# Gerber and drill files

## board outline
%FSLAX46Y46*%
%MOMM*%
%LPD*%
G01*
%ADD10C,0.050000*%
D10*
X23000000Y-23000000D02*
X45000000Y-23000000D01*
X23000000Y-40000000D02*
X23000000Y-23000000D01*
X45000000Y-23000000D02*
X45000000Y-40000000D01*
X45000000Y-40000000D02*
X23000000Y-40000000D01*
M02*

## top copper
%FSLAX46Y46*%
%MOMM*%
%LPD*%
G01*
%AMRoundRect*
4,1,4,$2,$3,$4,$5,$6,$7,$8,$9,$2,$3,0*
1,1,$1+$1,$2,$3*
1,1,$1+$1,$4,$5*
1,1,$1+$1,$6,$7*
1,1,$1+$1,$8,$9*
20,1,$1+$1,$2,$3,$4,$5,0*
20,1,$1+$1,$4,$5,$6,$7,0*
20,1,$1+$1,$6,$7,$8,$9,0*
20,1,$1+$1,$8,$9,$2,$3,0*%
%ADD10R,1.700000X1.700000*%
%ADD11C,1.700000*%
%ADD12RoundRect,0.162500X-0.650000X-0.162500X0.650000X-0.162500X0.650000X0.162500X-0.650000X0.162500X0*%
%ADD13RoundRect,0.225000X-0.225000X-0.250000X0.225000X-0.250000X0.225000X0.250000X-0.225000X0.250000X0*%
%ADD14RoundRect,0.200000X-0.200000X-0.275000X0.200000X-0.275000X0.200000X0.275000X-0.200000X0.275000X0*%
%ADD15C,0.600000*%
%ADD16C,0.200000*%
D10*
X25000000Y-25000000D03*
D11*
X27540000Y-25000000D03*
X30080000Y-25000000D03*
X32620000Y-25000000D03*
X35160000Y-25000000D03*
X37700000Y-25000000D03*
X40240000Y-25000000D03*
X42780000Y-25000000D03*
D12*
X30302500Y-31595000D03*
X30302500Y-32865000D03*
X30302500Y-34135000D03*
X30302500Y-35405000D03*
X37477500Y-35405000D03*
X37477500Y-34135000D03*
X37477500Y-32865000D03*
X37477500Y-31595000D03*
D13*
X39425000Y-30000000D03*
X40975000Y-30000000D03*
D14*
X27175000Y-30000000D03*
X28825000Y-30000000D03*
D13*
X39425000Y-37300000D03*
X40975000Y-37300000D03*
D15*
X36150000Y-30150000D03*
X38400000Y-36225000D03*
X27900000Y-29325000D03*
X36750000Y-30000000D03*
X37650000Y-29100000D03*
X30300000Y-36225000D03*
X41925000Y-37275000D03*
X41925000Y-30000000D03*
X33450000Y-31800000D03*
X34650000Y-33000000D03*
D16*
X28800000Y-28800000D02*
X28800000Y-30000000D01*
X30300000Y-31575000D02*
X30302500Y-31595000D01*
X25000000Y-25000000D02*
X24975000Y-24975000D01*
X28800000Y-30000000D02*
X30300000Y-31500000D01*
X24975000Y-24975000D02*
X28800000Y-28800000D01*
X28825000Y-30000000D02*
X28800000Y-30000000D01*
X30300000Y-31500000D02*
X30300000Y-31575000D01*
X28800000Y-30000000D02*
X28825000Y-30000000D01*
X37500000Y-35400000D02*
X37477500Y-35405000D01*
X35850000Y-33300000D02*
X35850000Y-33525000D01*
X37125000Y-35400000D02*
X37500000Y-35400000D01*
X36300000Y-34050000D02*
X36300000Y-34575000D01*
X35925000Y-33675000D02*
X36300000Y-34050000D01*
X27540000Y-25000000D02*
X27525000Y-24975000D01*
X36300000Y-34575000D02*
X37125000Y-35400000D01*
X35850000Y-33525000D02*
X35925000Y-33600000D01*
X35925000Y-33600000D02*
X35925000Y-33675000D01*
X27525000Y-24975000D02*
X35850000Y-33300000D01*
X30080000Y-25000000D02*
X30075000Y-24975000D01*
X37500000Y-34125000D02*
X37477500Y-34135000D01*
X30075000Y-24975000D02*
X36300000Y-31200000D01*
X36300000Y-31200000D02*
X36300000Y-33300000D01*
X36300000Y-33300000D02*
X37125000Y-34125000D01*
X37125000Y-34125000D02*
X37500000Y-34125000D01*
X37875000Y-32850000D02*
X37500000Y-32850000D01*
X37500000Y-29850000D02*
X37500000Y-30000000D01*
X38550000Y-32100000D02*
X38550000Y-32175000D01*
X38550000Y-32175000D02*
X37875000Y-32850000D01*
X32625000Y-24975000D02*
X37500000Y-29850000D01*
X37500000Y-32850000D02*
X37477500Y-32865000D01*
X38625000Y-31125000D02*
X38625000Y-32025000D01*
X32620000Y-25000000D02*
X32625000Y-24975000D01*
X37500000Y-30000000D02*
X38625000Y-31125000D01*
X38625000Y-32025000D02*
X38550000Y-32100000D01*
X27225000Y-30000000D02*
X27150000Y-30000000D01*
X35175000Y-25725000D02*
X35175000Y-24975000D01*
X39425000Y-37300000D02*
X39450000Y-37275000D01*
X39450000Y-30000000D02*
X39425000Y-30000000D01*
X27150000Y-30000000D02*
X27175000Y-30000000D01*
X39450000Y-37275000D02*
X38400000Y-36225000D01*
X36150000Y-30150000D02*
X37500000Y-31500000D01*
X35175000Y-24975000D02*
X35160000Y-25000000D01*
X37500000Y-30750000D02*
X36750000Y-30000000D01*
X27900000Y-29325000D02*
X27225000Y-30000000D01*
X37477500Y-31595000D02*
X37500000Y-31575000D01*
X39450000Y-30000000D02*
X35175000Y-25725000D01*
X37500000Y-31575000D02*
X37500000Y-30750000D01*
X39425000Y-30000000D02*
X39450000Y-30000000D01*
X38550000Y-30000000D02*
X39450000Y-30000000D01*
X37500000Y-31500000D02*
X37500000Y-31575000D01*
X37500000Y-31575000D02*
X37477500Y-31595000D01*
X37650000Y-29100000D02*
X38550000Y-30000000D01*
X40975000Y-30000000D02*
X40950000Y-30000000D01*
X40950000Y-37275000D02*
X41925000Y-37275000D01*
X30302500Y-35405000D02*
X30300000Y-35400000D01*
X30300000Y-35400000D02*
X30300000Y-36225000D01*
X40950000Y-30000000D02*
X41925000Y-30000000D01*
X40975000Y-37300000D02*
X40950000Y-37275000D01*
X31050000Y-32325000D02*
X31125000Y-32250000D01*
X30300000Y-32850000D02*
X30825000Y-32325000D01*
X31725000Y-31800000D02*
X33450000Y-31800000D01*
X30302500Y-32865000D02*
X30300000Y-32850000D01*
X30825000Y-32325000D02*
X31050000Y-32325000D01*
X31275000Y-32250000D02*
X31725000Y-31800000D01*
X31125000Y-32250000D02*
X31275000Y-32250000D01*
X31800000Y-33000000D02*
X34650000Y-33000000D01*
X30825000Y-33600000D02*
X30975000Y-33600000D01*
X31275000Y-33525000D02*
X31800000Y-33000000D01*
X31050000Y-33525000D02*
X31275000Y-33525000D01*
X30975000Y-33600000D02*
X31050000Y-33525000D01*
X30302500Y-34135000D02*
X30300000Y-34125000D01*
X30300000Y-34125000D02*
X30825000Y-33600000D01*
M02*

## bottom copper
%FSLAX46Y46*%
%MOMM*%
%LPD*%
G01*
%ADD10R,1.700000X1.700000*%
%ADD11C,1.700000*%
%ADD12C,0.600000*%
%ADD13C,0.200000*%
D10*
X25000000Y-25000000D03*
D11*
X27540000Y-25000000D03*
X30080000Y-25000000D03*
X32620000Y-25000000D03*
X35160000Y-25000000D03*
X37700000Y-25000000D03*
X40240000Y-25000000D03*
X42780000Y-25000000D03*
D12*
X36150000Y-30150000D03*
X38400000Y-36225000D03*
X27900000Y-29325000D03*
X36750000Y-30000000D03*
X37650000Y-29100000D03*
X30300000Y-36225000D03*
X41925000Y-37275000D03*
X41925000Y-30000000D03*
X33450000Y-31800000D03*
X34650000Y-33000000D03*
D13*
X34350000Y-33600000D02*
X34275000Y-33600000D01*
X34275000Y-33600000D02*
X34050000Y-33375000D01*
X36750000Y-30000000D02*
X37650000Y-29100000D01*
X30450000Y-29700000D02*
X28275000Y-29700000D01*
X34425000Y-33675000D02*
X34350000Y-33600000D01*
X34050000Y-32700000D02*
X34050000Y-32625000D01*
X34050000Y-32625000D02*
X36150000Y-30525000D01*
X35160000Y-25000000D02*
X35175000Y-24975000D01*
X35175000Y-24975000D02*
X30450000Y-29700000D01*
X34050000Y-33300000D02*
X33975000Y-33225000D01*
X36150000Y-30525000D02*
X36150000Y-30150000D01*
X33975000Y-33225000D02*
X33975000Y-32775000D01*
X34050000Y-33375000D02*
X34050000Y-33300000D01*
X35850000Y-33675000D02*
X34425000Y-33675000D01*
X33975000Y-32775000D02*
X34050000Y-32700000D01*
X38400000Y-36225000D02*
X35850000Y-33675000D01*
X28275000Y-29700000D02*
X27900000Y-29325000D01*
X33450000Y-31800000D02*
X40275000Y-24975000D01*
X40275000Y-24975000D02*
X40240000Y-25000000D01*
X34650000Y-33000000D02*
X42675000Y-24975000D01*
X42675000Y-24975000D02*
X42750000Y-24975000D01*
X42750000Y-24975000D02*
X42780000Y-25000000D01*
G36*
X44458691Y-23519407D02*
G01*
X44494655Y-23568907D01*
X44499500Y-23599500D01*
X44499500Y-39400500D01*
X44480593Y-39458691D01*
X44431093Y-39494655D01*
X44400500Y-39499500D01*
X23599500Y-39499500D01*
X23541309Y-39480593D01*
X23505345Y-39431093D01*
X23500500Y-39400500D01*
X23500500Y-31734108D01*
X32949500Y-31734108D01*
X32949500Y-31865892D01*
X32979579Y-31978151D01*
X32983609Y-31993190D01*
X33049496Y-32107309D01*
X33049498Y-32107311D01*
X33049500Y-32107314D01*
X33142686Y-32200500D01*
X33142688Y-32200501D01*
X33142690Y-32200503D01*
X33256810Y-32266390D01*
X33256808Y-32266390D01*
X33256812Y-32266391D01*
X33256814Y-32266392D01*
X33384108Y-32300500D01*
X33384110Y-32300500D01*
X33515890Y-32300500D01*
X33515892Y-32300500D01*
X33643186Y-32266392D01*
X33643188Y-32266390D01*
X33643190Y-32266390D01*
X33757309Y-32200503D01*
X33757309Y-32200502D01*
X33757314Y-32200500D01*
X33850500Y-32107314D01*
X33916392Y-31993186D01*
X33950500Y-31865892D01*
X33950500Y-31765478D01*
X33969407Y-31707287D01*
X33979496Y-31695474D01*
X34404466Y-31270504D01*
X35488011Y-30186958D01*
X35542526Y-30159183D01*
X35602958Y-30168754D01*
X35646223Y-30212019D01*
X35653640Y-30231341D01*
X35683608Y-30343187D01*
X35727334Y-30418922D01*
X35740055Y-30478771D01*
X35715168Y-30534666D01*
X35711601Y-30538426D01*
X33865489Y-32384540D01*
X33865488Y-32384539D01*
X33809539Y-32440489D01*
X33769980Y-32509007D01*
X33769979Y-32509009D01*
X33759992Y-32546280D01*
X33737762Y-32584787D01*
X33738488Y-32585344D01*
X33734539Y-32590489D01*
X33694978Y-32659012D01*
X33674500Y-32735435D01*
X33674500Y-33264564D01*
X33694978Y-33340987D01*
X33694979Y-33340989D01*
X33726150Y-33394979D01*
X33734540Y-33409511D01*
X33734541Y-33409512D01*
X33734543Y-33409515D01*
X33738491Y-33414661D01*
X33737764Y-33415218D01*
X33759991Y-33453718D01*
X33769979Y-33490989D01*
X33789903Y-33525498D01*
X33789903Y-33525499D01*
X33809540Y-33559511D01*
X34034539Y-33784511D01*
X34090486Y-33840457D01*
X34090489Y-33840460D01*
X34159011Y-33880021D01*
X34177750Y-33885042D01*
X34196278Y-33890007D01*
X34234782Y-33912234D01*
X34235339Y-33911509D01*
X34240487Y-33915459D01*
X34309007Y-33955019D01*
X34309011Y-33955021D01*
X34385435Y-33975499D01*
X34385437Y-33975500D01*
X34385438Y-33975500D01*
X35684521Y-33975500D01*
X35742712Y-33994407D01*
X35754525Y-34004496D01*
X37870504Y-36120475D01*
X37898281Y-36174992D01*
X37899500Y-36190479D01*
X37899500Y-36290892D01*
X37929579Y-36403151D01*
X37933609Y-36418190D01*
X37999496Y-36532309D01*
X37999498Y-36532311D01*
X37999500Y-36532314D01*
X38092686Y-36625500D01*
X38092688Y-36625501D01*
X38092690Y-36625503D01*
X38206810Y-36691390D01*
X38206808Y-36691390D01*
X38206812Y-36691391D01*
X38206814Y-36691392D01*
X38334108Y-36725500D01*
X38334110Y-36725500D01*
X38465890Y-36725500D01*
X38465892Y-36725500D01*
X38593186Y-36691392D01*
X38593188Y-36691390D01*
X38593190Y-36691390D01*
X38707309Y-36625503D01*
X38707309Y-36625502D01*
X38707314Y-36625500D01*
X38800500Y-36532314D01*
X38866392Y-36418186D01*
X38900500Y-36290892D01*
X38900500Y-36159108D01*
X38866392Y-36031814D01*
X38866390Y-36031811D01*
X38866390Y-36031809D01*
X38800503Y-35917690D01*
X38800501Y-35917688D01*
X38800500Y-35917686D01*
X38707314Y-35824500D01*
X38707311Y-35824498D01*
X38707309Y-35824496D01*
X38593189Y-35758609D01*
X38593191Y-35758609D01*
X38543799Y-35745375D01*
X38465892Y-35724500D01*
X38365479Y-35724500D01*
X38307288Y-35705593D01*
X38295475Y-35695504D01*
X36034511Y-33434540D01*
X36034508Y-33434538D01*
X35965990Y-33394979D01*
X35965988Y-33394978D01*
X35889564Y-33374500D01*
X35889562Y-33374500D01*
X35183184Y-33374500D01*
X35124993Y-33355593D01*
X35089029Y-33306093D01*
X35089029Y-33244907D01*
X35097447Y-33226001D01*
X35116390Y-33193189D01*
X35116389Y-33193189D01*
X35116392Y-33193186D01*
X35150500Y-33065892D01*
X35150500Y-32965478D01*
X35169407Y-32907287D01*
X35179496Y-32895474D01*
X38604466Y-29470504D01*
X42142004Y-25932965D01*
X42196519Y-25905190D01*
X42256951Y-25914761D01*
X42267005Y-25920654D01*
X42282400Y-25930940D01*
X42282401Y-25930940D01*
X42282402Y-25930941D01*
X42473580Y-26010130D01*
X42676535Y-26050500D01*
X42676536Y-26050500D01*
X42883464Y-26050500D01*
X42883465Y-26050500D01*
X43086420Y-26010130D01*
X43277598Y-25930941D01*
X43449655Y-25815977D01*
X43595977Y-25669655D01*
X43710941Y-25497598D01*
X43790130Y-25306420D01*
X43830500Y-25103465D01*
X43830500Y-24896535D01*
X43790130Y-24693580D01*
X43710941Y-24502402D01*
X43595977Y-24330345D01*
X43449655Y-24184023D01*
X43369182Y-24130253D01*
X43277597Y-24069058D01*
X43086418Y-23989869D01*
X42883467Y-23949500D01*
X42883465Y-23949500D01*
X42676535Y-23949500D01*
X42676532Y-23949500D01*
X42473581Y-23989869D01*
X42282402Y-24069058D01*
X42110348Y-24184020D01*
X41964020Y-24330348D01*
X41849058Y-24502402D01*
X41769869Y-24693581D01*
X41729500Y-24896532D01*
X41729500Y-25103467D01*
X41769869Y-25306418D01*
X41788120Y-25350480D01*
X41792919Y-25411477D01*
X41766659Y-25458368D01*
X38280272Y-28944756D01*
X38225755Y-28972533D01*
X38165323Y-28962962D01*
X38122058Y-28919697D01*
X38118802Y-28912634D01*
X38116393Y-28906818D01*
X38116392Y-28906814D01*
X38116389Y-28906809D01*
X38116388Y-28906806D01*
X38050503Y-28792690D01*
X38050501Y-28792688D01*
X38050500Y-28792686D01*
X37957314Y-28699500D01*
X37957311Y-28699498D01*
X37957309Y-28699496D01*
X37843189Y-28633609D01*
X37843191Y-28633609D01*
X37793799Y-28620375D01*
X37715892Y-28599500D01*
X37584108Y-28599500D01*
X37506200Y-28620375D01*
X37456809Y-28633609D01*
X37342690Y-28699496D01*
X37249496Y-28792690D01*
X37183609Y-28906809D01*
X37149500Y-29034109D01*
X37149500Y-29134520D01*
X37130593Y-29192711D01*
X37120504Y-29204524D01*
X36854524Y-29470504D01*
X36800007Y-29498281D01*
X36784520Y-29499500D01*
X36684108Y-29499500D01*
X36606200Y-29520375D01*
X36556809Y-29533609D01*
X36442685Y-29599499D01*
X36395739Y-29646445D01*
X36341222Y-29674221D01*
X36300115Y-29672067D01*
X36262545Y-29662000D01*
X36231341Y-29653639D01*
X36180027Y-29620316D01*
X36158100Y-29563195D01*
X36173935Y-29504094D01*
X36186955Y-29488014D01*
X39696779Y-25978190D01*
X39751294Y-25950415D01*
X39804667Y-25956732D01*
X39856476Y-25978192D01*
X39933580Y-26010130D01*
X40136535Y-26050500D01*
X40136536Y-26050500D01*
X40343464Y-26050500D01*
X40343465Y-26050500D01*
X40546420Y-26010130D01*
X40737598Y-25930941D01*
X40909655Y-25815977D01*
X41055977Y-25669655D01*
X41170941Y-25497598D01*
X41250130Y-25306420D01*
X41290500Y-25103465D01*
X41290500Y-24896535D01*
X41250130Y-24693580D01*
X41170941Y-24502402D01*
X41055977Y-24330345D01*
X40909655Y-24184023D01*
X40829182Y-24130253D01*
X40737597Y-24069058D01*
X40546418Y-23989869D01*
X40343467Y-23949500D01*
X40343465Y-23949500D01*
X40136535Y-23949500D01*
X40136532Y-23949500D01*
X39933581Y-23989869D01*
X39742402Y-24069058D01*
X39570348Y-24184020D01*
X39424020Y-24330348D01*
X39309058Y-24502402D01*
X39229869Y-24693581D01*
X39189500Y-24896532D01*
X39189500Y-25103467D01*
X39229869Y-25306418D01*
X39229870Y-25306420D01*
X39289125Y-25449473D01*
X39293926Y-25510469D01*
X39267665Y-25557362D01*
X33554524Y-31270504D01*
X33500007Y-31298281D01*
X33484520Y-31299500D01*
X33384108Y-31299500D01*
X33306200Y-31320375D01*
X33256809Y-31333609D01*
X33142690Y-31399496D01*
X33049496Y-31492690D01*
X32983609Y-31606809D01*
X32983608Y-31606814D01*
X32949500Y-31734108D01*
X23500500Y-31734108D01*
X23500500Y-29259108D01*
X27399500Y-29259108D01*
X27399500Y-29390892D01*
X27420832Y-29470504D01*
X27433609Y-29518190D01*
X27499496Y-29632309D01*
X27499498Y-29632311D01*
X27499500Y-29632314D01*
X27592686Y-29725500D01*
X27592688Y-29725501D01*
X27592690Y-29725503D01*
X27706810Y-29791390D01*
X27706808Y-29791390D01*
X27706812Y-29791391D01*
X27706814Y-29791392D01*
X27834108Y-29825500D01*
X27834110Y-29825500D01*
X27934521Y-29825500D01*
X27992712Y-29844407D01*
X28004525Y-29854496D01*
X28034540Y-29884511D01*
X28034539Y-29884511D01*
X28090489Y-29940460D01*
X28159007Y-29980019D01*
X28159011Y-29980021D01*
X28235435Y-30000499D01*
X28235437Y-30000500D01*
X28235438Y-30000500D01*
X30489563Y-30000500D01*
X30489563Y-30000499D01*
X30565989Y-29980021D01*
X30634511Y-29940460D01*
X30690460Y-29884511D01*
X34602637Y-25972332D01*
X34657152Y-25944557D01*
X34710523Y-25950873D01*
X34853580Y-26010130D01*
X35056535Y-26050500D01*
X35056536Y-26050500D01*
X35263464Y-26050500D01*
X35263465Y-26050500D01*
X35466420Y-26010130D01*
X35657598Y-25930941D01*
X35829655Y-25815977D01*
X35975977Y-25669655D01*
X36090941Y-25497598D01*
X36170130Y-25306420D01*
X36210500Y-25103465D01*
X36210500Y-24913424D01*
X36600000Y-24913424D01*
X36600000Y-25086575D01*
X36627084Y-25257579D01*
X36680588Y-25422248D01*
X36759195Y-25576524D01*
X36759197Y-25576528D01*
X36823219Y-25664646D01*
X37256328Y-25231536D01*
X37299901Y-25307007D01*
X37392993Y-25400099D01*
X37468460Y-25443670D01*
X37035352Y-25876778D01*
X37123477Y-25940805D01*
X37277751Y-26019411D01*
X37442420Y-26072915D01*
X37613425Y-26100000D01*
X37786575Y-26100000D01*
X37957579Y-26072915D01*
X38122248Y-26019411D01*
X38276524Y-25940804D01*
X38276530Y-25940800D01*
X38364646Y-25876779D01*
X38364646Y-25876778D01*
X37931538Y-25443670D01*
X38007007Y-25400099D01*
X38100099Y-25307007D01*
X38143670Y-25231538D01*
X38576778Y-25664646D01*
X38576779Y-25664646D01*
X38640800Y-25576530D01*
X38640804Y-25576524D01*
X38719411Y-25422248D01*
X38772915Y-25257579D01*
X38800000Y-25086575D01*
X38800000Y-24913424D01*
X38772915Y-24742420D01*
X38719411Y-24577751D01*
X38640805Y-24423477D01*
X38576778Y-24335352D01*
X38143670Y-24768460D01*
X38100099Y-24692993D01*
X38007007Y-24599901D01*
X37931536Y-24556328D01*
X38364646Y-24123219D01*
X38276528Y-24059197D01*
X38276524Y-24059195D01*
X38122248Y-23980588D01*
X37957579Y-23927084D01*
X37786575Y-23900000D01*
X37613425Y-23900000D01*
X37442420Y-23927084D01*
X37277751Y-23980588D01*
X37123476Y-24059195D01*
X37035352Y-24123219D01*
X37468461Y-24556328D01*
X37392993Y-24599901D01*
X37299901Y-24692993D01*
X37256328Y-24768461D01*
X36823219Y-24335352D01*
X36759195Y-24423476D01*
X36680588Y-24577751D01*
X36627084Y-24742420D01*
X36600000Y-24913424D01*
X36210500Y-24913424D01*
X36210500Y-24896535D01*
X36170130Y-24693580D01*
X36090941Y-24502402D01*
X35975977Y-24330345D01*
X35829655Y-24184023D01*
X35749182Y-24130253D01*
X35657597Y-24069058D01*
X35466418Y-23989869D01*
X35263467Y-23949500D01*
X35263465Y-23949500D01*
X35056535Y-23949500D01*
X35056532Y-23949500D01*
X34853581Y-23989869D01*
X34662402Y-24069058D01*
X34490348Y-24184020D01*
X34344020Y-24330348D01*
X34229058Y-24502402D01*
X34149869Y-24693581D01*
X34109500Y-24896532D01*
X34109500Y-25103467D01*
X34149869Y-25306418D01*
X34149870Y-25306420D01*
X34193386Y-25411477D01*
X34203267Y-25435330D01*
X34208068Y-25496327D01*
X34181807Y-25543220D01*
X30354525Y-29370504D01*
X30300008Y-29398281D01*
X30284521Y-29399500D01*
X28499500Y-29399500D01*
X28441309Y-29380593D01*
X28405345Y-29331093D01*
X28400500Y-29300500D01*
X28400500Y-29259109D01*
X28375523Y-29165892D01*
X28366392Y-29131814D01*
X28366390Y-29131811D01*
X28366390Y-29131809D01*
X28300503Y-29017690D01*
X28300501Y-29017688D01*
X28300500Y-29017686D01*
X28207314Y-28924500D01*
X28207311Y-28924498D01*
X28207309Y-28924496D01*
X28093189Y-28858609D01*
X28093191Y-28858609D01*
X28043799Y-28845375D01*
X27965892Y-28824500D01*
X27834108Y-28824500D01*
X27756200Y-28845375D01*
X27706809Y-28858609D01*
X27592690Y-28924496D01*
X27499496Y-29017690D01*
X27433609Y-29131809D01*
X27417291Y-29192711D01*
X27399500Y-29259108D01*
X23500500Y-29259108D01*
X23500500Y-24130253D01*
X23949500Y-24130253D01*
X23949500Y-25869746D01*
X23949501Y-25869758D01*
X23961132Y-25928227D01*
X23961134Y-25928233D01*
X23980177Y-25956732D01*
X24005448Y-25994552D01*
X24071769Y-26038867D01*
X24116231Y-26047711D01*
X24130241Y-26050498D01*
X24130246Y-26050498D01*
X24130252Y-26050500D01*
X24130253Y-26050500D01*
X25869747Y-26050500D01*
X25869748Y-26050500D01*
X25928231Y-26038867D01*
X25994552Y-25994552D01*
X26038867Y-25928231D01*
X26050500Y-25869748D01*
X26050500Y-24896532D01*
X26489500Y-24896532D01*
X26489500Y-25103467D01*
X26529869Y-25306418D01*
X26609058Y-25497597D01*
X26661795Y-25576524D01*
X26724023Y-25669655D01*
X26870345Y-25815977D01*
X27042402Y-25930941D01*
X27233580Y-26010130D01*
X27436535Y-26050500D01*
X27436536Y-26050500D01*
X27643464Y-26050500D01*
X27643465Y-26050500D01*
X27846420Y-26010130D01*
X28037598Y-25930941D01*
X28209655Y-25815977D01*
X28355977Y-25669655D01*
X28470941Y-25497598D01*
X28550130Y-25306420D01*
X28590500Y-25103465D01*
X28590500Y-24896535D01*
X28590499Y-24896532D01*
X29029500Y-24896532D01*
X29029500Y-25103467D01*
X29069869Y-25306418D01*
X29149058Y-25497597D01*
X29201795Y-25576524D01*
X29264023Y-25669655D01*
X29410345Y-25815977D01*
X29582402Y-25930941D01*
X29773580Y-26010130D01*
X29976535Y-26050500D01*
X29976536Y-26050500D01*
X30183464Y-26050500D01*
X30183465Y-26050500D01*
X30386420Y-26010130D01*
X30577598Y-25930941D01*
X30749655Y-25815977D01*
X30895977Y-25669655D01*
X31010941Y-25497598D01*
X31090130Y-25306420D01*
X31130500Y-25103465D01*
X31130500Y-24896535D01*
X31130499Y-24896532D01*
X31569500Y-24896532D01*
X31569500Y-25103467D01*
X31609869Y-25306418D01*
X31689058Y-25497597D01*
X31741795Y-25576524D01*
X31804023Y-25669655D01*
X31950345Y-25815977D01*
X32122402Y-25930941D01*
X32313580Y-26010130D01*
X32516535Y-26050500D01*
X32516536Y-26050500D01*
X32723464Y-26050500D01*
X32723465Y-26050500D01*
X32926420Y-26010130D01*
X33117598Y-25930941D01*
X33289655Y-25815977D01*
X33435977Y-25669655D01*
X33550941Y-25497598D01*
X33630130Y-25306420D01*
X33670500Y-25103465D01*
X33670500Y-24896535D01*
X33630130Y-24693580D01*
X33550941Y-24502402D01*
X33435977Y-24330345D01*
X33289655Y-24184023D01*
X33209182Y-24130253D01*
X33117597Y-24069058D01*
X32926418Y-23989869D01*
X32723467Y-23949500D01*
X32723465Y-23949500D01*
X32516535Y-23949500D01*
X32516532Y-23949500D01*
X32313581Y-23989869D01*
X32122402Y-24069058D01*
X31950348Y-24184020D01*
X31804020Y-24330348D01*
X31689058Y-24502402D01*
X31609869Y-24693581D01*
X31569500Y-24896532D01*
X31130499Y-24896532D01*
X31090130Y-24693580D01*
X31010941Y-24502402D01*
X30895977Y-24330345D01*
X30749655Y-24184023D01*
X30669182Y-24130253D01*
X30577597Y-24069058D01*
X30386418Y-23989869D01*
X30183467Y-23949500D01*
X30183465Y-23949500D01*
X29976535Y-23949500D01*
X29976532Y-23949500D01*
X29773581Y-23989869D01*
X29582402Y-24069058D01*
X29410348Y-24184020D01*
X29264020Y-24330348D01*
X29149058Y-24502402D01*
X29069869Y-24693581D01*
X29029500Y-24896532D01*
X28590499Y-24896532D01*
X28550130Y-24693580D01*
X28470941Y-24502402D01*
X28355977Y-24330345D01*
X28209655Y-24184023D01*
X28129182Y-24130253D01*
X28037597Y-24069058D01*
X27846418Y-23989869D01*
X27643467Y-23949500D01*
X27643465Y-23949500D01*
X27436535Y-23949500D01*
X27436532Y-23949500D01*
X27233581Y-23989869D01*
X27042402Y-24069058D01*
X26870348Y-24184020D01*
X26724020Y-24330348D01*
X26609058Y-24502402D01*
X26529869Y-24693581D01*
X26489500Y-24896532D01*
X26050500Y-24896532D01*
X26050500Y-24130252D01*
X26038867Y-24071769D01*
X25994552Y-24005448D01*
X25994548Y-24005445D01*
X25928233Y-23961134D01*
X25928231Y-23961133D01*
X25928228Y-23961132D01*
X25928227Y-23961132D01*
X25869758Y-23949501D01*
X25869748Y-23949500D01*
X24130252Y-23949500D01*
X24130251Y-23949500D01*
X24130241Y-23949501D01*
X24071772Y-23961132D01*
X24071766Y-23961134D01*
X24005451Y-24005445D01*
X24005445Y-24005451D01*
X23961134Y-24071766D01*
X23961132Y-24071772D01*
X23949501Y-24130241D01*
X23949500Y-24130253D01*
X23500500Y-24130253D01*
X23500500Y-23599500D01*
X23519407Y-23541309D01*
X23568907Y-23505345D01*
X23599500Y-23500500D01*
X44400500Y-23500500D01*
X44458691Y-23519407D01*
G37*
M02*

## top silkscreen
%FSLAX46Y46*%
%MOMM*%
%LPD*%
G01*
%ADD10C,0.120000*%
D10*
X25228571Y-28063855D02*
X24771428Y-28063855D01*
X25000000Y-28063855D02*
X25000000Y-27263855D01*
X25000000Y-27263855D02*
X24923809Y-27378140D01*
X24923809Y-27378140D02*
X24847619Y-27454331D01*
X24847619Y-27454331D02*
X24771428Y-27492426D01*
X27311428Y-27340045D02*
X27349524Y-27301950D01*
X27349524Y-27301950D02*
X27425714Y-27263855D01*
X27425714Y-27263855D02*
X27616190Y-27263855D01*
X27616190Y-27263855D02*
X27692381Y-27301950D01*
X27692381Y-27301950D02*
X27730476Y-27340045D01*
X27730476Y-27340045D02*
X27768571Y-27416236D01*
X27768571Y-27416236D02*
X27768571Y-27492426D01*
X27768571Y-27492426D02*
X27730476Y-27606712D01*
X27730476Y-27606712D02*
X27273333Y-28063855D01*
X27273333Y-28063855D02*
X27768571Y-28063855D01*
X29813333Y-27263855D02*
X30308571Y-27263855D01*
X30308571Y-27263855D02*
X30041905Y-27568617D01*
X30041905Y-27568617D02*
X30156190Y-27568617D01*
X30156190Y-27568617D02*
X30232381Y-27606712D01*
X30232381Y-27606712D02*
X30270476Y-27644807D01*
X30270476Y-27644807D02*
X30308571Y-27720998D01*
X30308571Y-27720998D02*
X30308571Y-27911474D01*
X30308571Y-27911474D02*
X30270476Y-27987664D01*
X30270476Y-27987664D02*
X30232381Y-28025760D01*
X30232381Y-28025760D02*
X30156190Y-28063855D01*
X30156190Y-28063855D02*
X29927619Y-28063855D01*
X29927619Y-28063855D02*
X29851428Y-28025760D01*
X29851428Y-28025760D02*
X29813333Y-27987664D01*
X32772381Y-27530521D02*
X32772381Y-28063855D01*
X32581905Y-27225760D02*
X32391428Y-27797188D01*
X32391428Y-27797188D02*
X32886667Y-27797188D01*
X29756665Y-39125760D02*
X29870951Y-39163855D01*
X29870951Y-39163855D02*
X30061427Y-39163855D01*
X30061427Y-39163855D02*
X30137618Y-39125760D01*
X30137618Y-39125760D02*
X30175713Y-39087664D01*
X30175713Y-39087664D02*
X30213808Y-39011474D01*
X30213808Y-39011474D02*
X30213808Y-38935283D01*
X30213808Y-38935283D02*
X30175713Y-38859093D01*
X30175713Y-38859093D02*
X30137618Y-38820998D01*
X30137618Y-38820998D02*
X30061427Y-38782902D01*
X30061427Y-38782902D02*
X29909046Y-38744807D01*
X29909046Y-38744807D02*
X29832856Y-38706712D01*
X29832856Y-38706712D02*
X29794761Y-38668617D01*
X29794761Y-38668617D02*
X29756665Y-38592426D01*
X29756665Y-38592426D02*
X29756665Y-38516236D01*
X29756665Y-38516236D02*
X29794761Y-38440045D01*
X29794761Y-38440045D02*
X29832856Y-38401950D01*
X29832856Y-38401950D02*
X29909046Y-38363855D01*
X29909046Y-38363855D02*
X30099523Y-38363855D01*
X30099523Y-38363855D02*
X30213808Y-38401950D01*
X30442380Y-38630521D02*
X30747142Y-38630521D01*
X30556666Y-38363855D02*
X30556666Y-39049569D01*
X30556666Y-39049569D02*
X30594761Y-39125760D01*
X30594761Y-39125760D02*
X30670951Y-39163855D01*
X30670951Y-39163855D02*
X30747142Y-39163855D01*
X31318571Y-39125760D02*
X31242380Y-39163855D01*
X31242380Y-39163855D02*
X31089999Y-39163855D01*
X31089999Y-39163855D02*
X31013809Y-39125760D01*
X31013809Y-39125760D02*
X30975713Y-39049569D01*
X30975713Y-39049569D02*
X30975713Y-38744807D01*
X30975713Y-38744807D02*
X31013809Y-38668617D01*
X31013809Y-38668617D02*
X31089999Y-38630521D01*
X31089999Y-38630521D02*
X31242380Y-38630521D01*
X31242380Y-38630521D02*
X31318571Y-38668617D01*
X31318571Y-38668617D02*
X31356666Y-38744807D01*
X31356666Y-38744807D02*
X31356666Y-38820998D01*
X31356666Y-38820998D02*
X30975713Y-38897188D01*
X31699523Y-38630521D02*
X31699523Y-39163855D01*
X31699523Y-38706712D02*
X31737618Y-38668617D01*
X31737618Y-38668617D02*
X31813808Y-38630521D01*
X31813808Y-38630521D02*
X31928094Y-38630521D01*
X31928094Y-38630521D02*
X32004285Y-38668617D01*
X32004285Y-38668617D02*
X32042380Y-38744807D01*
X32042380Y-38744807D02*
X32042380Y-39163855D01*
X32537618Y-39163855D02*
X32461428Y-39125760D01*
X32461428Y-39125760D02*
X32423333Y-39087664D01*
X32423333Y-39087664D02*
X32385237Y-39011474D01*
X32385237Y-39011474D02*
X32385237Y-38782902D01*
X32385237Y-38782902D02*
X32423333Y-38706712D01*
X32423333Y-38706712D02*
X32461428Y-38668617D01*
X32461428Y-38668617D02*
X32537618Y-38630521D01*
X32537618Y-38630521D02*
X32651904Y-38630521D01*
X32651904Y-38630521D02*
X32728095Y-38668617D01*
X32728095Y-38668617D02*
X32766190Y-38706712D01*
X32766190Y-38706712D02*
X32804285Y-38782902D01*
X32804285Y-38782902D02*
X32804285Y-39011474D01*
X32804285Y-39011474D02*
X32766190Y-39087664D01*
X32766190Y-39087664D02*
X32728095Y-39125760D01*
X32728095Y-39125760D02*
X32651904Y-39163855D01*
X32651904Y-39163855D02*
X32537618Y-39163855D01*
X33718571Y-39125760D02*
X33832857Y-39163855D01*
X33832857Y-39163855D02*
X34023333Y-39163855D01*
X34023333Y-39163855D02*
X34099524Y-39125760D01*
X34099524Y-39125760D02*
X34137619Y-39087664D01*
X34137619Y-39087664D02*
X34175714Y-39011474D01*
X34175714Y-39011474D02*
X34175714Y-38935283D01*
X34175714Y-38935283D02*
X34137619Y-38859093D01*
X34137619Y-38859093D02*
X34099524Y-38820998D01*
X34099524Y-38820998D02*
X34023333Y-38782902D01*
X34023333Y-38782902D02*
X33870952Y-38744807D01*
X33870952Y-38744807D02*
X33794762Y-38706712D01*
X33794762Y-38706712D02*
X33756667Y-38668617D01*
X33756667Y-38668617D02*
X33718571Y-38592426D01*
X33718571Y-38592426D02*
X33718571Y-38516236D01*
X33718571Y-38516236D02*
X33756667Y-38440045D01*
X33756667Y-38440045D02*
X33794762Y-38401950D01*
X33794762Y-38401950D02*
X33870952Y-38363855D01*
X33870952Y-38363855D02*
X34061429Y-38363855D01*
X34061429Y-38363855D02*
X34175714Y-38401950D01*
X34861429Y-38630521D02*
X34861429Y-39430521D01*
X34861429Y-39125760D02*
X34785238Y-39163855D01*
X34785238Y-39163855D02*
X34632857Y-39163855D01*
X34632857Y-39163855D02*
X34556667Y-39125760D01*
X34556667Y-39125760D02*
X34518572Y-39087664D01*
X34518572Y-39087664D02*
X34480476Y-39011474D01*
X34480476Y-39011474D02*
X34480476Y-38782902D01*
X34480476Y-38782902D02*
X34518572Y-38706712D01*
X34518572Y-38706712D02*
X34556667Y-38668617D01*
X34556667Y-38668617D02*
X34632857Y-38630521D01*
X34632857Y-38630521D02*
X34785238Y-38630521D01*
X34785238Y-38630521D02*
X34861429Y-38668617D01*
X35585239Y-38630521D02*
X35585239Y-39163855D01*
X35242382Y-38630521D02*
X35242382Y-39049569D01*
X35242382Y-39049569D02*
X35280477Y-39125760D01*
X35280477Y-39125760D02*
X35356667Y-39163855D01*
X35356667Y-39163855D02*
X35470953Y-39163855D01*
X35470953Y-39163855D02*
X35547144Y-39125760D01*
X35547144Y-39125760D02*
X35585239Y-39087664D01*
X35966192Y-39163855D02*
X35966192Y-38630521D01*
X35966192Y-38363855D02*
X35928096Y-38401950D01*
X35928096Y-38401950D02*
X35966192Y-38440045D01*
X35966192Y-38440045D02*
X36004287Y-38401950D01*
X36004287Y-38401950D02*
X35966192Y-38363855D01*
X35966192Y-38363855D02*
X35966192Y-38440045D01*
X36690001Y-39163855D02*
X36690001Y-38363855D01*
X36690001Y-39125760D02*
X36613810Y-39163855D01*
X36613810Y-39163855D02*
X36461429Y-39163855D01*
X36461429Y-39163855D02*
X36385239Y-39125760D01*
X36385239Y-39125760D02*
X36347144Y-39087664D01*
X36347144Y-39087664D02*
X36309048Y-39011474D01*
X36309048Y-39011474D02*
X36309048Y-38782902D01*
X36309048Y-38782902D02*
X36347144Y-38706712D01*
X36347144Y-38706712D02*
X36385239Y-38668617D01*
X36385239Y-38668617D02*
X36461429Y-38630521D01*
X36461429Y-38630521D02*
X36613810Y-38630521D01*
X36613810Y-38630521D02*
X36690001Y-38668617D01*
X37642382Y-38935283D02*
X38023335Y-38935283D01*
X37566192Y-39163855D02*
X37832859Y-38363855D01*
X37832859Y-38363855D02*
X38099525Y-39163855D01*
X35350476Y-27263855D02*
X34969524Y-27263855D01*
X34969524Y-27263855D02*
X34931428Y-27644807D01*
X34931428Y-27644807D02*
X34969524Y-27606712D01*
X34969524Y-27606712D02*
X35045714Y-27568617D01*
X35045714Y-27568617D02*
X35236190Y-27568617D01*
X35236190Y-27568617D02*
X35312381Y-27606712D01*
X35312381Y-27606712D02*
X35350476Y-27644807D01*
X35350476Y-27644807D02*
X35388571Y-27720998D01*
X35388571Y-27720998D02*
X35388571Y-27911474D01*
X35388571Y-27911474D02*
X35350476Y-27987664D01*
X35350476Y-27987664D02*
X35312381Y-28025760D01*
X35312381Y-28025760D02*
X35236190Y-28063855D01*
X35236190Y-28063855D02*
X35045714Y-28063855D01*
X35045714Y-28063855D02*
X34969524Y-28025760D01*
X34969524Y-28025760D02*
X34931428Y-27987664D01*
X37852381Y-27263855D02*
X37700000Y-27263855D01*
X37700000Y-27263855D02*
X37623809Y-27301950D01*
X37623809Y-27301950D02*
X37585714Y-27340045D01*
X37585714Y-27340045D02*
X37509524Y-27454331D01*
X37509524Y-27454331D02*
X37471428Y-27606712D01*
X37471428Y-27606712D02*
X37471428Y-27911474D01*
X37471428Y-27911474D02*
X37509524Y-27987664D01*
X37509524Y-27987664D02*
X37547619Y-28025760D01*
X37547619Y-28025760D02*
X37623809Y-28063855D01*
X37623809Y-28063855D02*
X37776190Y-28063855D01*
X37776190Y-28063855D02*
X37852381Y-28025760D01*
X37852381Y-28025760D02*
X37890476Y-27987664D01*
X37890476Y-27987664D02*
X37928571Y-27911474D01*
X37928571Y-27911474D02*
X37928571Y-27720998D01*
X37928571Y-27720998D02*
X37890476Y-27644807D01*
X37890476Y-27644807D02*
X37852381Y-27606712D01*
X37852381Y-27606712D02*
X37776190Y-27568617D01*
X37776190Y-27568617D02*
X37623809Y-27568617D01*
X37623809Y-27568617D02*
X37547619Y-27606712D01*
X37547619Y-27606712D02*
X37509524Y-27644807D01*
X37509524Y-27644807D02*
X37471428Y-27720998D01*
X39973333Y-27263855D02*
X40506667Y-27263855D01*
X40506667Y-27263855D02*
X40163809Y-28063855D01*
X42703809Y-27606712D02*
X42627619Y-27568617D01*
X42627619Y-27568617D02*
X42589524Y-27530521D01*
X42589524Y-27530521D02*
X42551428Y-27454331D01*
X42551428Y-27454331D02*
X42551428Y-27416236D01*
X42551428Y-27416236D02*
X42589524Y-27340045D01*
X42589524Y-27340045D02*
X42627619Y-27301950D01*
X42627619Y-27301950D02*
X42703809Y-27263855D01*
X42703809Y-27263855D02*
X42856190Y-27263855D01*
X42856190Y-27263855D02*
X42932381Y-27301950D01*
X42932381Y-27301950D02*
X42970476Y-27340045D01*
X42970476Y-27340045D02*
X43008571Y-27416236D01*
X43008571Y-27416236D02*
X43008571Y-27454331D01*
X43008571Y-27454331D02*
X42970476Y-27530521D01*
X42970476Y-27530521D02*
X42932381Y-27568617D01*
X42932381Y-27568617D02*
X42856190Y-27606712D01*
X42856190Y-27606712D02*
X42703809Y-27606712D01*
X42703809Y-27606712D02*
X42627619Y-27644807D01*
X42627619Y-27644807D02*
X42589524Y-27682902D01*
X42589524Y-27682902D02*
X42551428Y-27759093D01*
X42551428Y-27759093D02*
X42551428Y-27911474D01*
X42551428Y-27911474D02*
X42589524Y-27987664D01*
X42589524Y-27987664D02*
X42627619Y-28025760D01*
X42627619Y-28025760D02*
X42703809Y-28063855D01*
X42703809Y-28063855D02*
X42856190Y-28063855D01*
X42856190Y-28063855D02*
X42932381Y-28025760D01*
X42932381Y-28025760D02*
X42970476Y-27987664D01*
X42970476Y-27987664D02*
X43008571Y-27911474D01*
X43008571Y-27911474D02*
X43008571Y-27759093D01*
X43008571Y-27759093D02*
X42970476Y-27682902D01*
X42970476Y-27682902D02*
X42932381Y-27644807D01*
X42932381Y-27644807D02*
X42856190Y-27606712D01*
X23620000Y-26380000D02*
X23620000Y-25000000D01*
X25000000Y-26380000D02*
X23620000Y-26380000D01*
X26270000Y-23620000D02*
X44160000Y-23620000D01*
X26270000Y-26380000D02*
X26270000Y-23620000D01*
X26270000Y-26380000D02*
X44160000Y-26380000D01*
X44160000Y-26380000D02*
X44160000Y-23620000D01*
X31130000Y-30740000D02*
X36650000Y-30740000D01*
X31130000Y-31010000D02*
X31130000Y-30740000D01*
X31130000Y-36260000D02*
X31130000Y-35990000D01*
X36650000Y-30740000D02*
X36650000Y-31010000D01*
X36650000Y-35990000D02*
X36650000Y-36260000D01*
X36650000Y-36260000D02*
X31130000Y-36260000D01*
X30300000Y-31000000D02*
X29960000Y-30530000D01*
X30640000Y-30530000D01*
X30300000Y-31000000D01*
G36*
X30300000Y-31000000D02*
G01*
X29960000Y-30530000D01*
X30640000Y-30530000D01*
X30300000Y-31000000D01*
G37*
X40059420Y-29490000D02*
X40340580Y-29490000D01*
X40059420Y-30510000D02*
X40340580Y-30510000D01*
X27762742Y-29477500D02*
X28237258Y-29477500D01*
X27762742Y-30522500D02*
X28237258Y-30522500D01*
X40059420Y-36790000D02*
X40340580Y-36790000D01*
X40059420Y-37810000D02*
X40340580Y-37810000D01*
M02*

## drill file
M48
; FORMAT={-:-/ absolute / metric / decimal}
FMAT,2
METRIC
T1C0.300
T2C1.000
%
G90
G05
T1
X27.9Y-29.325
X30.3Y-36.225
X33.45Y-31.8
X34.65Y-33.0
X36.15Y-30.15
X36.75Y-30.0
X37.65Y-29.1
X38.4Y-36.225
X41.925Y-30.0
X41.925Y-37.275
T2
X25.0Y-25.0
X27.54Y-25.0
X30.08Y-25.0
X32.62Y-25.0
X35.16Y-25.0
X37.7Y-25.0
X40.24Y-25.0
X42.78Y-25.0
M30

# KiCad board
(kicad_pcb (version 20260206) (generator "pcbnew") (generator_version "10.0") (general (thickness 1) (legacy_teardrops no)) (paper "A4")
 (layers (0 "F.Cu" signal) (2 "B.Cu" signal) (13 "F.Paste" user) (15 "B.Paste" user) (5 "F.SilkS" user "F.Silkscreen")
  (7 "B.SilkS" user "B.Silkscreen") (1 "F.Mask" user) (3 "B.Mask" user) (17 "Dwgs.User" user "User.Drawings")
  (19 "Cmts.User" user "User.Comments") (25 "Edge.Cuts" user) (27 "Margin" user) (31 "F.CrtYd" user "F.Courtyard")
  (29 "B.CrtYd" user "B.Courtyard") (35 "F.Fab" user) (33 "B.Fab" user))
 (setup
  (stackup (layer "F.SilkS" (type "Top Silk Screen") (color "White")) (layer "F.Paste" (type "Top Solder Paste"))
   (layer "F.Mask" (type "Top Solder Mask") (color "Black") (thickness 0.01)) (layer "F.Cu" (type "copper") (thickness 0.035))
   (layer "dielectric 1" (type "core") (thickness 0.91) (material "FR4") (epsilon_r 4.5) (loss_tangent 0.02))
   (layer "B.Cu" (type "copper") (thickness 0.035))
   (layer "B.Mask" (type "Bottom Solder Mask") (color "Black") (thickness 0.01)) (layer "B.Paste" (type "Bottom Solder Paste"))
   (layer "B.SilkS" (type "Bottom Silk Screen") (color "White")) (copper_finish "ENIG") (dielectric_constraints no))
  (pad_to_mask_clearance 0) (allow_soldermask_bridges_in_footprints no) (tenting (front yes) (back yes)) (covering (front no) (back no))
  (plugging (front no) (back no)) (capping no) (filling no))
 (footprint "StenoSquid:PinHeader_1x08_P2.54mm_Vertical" (layer "F.Cu") (at 25 25 90)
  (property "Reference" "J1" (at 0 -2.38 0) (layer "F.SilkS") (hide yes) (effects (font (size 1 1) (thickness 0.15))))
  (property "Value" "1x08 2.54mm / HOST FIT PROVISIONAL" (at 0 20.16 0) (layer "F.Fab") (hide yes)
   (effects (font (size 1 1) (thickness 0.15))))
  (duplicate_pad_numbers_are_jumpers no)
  (fp_line (start -1.38 -1.38) (end 0 -1.38) (stroke (width 0.12) (type solid)) (layer "F.SilkS"))
  (fp_line (start -1.38 0) (end -1.38 -1.38) (stroke (width 0.12) (type solid)) (layer "F.SilkS"))
  (fp_line (start 1.38 1.27) (end 1.38 19.16) (stroke (width 0.12) (type solid)) (layer "F.SilkS"))
  (fp_line (start -1.38 1.27) (end 1.38 1.27) (stroke (width 0.12) (type solid)) (layer "F.SilkS"))
  (fp_line (start -1.38 1.27) (end -1.38 19.16) (stroke (width 0.12) (type solid)) (layer "F.SilkS"))
  (fp_line (start -1.38 19.16) (end 1.38 19.16) (stroke (width 0.12) (type solid)) (layer "F.SilkS"))
  (pad "1" thru_hole rect (at 0 0 90) (size 1.7 1.7) (drill 1) (layers "*.Cu" "*.Mask") (remove_unused_layers no) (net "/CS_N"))
  (pad "2" thru_hole circle (at 0 2.54 90) (size 1.7 1.7) (drill 1) (layers "*.Cu" "*.Mask") (remove_unused_layers no) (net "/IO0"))
  (pad "3" thru_hole circle (at 0 5.08 90) (size 1.7 1.7) (drill 1) (layers "*.Cu" "*.Mask") (remove_unused_layers no) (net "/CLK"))
  (pad "4" thru_hole circle (at 0 7.62 90) (size 1.7 1.7) (drill 1) (layers "*.Cu" "*.Mask") (remove_unused_layers no) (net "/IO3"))
  (pad "5" thru_hole circle (at 0 10.16 90) (size 1.7 1.7) (drill 1) (layers "*.Cu" "*.Mask") (remove_unused_layers no) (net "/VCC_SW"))
  (pad "6" thru_hole circle (at 0 12.7 90) (size 1.7 1.7) (drill 1) (layers "*.Cu" "*.Mask") (remove_unused_layers no) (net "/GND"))
  (pad "7" thru_hole circle (at 0 15.24 90) (size 1.7 1.7) (drill 1) (layers "*.Cu" "*.Mask") (remove_unused_layers no) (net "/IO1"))
  (pad "8" thru_hole circle (at 0 17.78 90) (size 1.7 1.7) (drill 1) (layers "*.Cu" "*.Mask") (remove_unused_layers no) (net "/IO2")))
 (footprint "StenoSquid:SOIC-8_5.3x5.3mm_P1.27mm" (layer "F.Cu") (at 33.89 33.5)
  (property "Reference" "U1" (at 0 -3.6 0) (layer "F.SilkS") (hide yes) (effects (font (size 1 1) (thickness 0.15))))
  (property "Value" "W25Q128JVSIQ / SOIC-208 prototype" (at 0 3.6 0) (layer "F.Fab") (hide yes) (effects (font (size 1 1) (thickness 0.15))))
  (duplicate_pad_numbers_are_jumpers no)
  (fp_line (start -2.76 -2.76) (end 2.76 -2.76) (stroke (width 0.12) (type solid)) (layer "F.SilkS"))
  (fp_line (start -2.76 -2.49) (end -2.76 -2.76) (stroke (width 0.12) (type solid)) (layer "F.SilkS"))
  (fp_line (start -2.76 2.76) (end -2.76 2.49) (stroke (width 0.12) (type solid)) (layer "F.SilkS"))
  (fp_line (start 2.76 -2.76) (end 2.76 -2.49) (stroke (width 0.12) (type solid)) (layer "F.SilkS"))
  (fp_line (start 2.76 2.49) (end 2.76 2.76) (stroke (width 0.12) (type solid)) (layer "F.SilkS"))
  (fp_line (start 2.76 2.76) (end -2.76 2.76) (stroke (width 0.12) (type solid)) (layer "F.SilkS"))
  (fp_poly (pts (xy -3.59 -2.5) (xy -3.93 -2.97) (xy -3.25 -2.97)) (stroke (width 0.12) (type solid)) (fill yes) (layer "F.SilkS"))
  (pad "1" smd roundrect (at -3.5875 -1.905) (size 1.625 0.65) (layers "F.Cu" "F.Mask" "F.Paste") (roundrect_rratio 0.25) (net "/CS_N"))
  (pad "2" smd roundrect (at -3.5875 -0.635) (size 1.625 0.65) (layers "F.Cu" "F.Mask" "F.Paste") (roundrect_rratio 0.25) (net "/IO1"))
  (pad "3" smd roundrect (at -3.5875 0.635) (size 1.625 0.65) (layers "F.Cu" "F.Mask" "F.Paste") (roundrect_rratio 0.25) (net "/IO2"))
  (pad "4" smd roundrect (at -3.5875 1.905) (size 1.625 0.65) (layers "F.Cu" "F.Mask" "F.Paste") (roundrect_rratio 0.25) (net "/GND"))
  (pad "5" smd roundrect (at 3.5875 1.905) (size 1.625 0.65) (layers "F.Cu" "F.Mask" "F.Paste") (roundrect_rratio 0.25) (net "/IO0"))
  (pad "6" smd roundrect (at 3.5875 0.635) (size 1.625 0.65) (layers "F.Cu" "F.Mask" "F.Paste") (roundrect_rratio 0.25) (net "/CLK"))
  (pad "7" smd roundrect (at 3.5875 -0.635) (size 1.625 0.65) (layers "F.Cu" "F.Mask" "F.Paste") (roundrect_rratio 0.25) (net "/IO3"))
  (pad "8" smd roundrect (at 3.5875 -1.905) (size 1.625 0.65) (layers "F.Cu" "F.Mask" "F.Paste") (roundrect_rratio 0.25) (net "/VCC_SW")))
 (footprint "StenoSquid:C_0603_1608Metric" (layer "F.Cu") (at 40.2 30)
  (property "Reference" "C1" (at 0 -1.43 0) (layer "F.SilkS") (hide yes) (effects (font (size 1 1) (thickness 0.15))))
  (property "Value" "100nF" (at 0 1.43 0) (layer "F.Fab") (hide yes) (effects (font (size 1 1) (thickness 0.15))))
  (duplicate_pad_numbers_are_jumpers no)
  (fp_line (start -0.14058 -0.51) (end 0.14058 -0.51) (stroke (width 0.12) (type solid)) (layer "F.SilkS"))
  (fp_line (start -0.14058 0.51) (end 0.14058 0.51) (stroke (width 0.12) (type solid)) (layer "F.SilkS"))
  (pad "1" smd roundrect (at -0.775 0) (size 0.9 0.95) (layers "F.Cu" "F.Mask" "F.Paste") (roundrect_rratio 0.25) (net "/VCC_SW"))
  (pad "2" smd roundrect (at 0.775 0) (size 0.9 0.95) (layers "F.Cu" "F.Mask" "F.Paste") (roundrect_rratio 0.25) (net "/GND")))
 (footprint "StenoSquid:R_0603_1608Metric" (layer "F.Cu") (at 28 30)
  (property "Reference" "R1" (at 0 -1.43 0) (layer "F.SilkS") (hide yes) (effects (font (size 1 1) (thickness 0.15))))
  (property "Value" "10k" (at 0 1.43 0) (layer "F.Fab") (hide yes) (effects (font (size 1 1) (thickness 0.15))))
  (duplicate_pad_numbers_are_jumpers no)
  (fp_line (start -0.237258 -0.5225) (end 0.237258 -0.5225) (stroke (width 0.12) (type solid)) (layer "F.SilkS"))
  (fp_line (start -0.237258 0.5225) (end 0.237258 0.5225) (stroke (width 0.12) (type solid)) (layer "F.SilkS"))
  (pad "1" smd roundrect (at -0.825 0) (size 0.8 0.95) (layers "F.Cu" "F.Mask" "F.Paste") (roundrect_rratio 0.25) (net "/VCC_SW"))
  (pad "2" smd roundrect (at 0.825 0) (size 0.8 0.95) (layers "F.Cu" "F.Mask" "F.Paste") (roundrect_rratio 0.25) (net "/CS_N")))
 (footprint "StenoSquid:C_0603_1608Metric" (layer "F.Cu") (at 40.2 37.3)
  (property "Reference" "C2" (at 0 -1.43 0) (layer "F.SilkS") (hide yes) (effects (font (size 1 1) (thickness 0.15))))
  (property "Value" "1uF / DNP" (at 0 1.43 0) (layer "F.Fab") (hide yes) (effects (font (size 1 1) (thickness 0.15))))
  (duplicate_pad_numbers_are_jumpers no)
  (fp_line (start -0.14058 -0.51) (end 0.14058 -0.51) (stroke (width 0.12) (type solid)) (layer "F.SilkS"))
  (fp_line (start -0.14058 0.51) (end 0.14058 0.51) (stroke (width 0.12) (type solid)) (layer "F.SilkS"))
  (pad "1" smd roundrect (at -0.775 0) (size 0.9 0.95) (layers "F.Cu" "F.Mask" "F.Paste") (roundrect_rratio 0.25) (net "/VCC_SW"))
  (pad "2" smd roundrect (at 0.775 0) (size 0.9 0.95) (layers "F.Cu" "F.Mask" "F.Paste") (roundrect_rratio 0.25) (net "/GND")))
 (gr_line (start 23 23) (end 45 23) (stroke (width 0.05) (type default)) (layer "Edge.Cuts"))
 (gr_line (start 23 40) (end 23 23) (stroke (width 0.05) (type default)) (layer "Edge.Cuts"))
 (gr_line (start 45 23) (end 45 40) (stroke (width 0.05) (type default)) (layer "Edge.Cuts"))
 (gr_line (start 45 40) (end 23 40) (stroke (width 0.05) (type default)) (layer "Edge.Cuts"))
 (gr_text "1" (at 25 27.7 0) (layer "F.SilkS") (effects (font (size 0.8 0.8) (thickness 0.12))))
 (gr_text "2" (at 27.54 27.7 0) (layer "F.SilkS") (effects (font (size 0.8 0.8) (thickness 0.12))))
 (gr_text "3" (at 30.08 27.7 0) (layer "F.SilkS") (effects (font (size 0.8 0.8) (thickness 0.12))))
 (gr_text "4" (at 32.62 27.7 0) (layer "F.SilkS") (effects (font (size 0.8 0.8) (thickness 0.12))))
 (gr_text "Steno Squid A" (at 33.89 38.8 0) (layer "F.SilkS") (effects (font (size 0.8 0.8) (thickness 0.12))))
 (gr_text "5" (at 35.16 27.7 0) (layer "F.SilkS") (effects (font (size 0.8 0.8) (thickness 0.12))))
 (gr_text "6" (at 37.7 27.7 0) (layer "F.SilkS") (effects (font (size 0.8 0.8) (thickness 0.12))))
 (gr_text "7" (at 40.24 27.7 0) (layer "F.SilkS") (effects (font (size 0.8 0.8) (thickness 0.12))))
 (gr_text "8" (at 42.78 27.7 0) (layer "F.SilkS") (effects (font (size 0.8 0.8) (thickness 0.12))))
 (segment (start 28.8 28.8) (end 28.8 30) (width 0.2) (layer "F.Cu") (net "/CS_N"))
 (segment (start 30.3 31.575) (end 30.3025 31.595) (width 0.2) (layer "F.Cu") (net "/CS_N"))
 (segment (start 25 25) (end 24.975 24.975) (width 0.2) (layer "F.Cu") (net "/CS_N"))
 (segment (start 28.8 30) (end 30.3 31.5) (width 0.2) (layer "F.Cu") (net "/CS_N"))
 (segment (start 24.975 24.975) (end 28.8 28.8) (width 0.2) (layer "F.Cu") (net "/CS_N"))
 (segment (start 28.825 30) (end 28.8 30) (width 0.2) (layer "F.Cu") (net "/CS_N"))
 (segment (start 30.3 31.5) (end 30.3 31.575) (width 0.2) (layer "F.Cu") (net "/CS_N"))
 (segment (start 28.8 30) (end 28.825 30) (width 0.2) (layer "F.Cu") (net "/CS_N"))
 (segment (start 37.5 35.4) (end 37.4775 35.405) (width 0.2) (layer "F.Cu") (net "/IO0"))
 (segment (start 35.85 33.3) (end 35.85 33.525) (width 0.2) (layer "F.Cu") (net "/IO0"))
 (segment (start 37.125 35.4) (end 37.5 35.4) (width 0.2) (layer "F.Cu") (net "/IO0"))
 (segment (start 36.3 34.05) (end 36.3 34.575) (width 0.2) (layer "F.Cu") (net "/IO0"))
 (segment (start 35.925 33.675) (end 36.3 34.05) (width 0.2) (layer "F.Cu") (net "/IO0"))
 (segment (start 27.54 25) (end 27.525 24.975) (width 0.2) (layer "F.Cu") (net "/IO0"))
 (segment (start 36.3 34.575) (end 37.125 35.4) (width 0.2) (layer "F.Cu") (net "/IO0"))
 (segment (start 35.85 33.525) (end 35.925 33.6) (width 0.2) (layer "F.Cu") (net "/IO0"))
 (segment (start 35.925 33.6) (end 35.925 33.675) (width 0.2) (layer "F.Cu") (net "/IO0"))
 (segment (start 27.525 24.975) (end 35.85 33.3) (width 0.2) (layer "F.Cu") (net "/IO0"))
 (segment (start 30.08 25) (end 30.075 24.975) (width 0.2) (layer "F.Cu") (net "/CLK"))
 (segment (start 37.5 34.125) (end 37.4775 34.135) (width 0.2) (layer "F.Cu") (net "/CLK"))
 (segment (start 30.075 24.975) (end 36.3 31.2) (width 0.2) (layer "F.Cu") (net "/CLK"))
 (segment (start 36.3 31.2) (end 36.3 33.3) (width 0.2) (layer "F.Cu") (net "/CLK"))
 (segment (start 36.3 33.3) (end 37.125 34.125) (width 0.2) (layer "F.Cu") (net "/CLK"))
 (segment (start 37.125 34.125) (end 37.5 34.125) (width 0.2) (layer "F.Cu") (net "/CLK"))
 (segment (start 37.875 32.85) (end 37.5 32.85) (width 0.2) (layer "F.Cu") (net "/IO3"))
 (segment (start 37.5 29.85) (end 37.5 30) (width 0.2) (layer "F.Cu") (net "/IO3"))
 (segment (start 38.55 32.1) (end 38.55 32.175) (width 0.2) (layer "F.Cu") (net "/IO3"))
 (segment (start 38.55 32.175) (end 37.875 32.85) (width 0.2) (layer "F.Cu") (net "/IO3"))
 (segment (start 32.625 24.975) (end 37.5 29.85) (width 0.2) (layer "F.Cu") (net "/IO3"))
 (segment (start 37.5 32.85) (end 37.4775 32.865) (width 0.2) (layer "F.Cu") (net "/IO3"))
 (segment (start 38.625 31.125) (end 38.625 32.025) (width 0.2) (layer "F.Cu") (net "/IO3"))
 (segment (start 32.62 25) (end 32.625 24.975) (width 0.2) (layer "F.Cu") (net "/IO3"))
 (segment (start 37.5 30) (end 38.625 31.125) (width 0.2) (layer "F.Cu") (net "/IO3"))
 (segment (start 38.625 32.025) (end 38.55 32.1) (width 0.2) (layer "F.Cu") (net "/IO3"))
 (segment (start 27.225 30) (end 27.15 30) (width 0.2) (layer "F.Cu") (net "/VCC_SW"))
 (segment (start 35.175 25.725) (end 35.175 24.975) (width 0.2) (layer "F.Cu") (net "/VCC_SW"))
 (segment (start 39.425 37.3) (end 39.45 37.275) (width 0.2) (layer "F.Cu") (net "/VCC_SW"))
 (segment (start 39.45 30) (end 39.425 30) (width 0.2) (layer "F.Cu") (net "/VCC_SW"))
 (segment (start 27.15 30) (end 27.175 30) (width 0.2) (layer "F.Cu") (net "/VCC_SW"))
 (segment (start 39.45 37.275) (end 38.4 36.225) (width 0.2) (layer "F.Cu") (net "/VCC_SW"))
 (segment (start 36.15 30.15) (end 37.5 31.5) (width 0.2) (layer "F.Cu") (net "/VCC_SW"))
 (segment (start 35.175 24.975) (end 35.16 25) (width 0.2) (layer "F.Cu") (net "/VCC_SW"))
 (segment (start 37.5 30.75) (end 36.75 30) (width 0.2) (layer "F.Cu") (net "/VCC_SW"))
 (segment (start 27.9 29.325) (end 27.225 30) (width 0.2) (layer "F.Cu") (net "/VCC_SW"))
 (segment (start 37.4775 31.595) (end 37.5 31.575) (width 0.2) (layer "F.Cu") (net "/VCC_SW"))
 (segment (start 39.45 30) (end 35.175 25.725) (width 0.2) (layer "F.Cu") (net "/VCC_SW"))
 (segment (start 37.5 31.575) (end 37.5 30.75) (width 0.2) (layer "F.Cu") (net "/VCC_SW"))
 (segment (start 39.425 30) (end 39.45 30) (width 0.2) (layer "F.Cu") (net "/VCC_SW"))
 (segment (start 38.55 30) (end 39.45 30) (width 0.2) (layer "F.Cu") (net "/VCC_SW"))
 (segment (start 37.5 31.5) (end 37.5 31.575) (width 0.2) (layer "F.Cu") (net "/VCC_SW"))
 (segment (start 37.5 31.575) (end 37.4775 31.595) (width 0.2) (layer "F.Cu") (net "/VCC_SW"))
 (segment (start 37.65 29.1) (end 38.55 30) (width 0.2) (layer "F.Cu") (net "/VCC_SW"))
 (via (at 36.15 30.15) (size 0.6) (drill 0.3) (layers "F.Cu" "B.Cu") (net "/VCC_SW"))
 (via (at 38.4 36.225) (size 0.6) (drill 0.3) (layers "F.Cu" "B.Cu") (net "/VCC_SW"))
 (via (at 27.9 29.325) (size 0.6) (drill 0.3) (layers "F.Cu" "B.Cu") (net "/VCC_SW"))
 (via (at 36.75 30) (size 0.6) (drill 0.3) (layers "F.Cu" "B.Cu") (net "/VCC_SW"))
 (via (at 37.65 29.1) (size 0.6) (drill 0.3) (layers "F.Cu" "B.Cu") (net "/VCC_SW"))
 (segment (start 34.35 33.6) (end 34.275 33.6) (width 0.2) (layer "B.Cu") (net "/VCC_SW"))
 (segment (start 34.275 33.6) (end 34.05 33.375) (width 0.2) (layer "B.Cu") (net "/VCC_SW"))
 (segment (start 36.75 30) (end 37.65 29.1) (width 0.2) (layer "B.Cu") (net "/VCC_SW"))
 (segment (start 30.45 29.7) (end 28.275 29.7) (width 0.2) (layer "B.Cu") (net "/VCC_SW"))
 (segment (start 34.425 33.675) (end 34.35 33.6) (width 0.2) (layer "B.Cu") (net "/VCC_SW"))
 (segment (start 34.05 32.7) (end 34.05 32.625) (width 0.2) (layer "B.Cu") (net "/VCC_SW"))
 (segment (start 34.05 32.625) (end 36.15 30.525) (width 0.2) (layer "B.Cu") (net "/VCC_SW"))
 (segment (start 35.16 25) (end 35.175 24.975) (width 0.2) (layer "B.Cu") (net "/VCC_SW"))
 (segment (start 35.175 24.975) (end 30.45 29.7) (width 0.2) (layer "B.Cu") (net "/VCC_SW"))
 (segment (start 34.05 33.3) (end 33.975 33.225) (width 0.2) (layer "B.Cu") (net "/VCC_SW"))
 (segment (start 36.15 30.525) (end 36.15 30.15) (width 0.2) (layer "B.Cu") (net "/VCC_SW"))
 (segment (start 33.975 33.225) (end 33.975 32.775) (width 0.2) (layer "B.Cu") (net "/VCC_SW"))
 (segment (start 34.05 33.375) (end 34.05 33.3) (width 0.2) (layer "B.Cu") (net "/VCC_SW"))
 (segment (start 35.85 33.675) (end 34.425 33.675) (width 0.2) (layer "B.Cu") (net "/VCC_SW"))
 (segment (start 33.975 32.775) (end 34.05 32.7) (width 0.2) (layer "B.Cu") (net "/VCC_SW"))
 (segment (start 38.4 36.225) (end 35.85 33.675) (width 0.2) (layer "B.Cu") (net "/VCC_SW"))
 (segment (start 28.275 29.7) (end 27.9 29.325) (width 0.2) (layer "B.Cu") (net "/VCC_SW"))
 (segment (start 40.975 30) (end 40.95 30) (width 0.2) (layer "F.Cu") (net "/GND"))
 (segment (start 40.95 37.275) (end 41.925 37.275) (width 0.2) (layer "F.Cu") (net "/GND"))
 (segment (start 30.3025 35.405) (end 30.3 35.4) (width 0.2) (layer "F.Cu") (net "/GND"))
 (segment (start 30.3 35.4) (end 30.3 36.225) (width 0.2) (layer "F.Cu") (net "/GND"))
 (segment (start 40.95 30) (end 41.925 30) (width 0.2) (layer "F.Cu") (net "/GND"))
 (segment (start 40.975 37.3) (end 40.95 37.275) (width 0.2) (layer "F.Cu") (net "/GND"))
 (via (at 30.3 36.225) (size 0.6) (drill 0.3) (layers "F.Cu" "B.Cu") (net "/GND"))
 (via (at 41.925 37.275) (size 0.6) (drill 0.3) (layers "F.Cu" "B.Cu") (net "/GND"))
 (via (at 41.925 30) (size 0.6) (drill 0.3) (layers "F.Cu" "B.Cu") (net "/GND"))
 (segment (start 31.05 32.325) (end 31.125 32.25) (width 0.2) (layer "F.Cu") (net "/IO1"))
 (segment (start 30.3 32.85) (end 30.825 32.325) (width 0.2) (layer "F.Cu") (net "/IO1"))
 (segment (start 31.725 31.8) (end 33.45 31.8) (width 0.2) (layer "F.Cu") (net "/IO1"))
 (segment (start 30.3025 32.865) (end 30.3 32.85) (width 0.2) (layer "F.Cu") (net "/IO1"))
 (segment (start 30.825 32.325) (end 31.05 32.325) (width 0.2) (layer "F.Cu") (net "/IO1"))
 (segment (start 31.275 32.25) (end 31.725 31.8) (width 0.2) (layer "F.Cu") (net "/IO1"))
 (segment (start 31.125 32.25) (end 31.275 32.25) (width 0.2) (layer "F.Cu") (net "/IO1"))
 (via (at 33.45 31.8) (size 0.6) (drill 0.3) (layers "F.Cu" "B.Cu") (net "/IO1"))
 (segment (start 33.45 31.8) (end 40.275 24.975) (width 0.2) (layer "B.Cu") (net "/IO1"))
 (segment (start 40.275 24.975) (end 40.24 25) (width 0.2) (layer "B.Cu") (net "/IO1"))
 (segment (start 31.8 33) (end 34.65 33) (width 0.2) (layer "F.Cu") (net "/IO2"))
 (segment (start 30.825 33.6) (end 30.975 33.6) (width 0.2) (layer "F.Cu") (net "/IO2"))
 (segment (start 31.275 33.525) (end 31.8 33) (width 0.2) (layer "F.Cu") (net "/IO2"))
 (segment (start 31.05 33.525) (end 31.275 33.525) (width 0.2) (layer "F.Cu") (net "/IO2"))
 (segment (start 30.975 33.6) (end 31.05 33.525) (width 0.2) (layer "F.Cu") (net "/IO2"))
 (segment (start 30.3025 34.135) (end 30.3 34.125) (width 0.2) (layer "F.Cu") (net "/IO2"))
 (segment (start 30.3 34.125) (end 30.825 33.6) (width 0.2) (layer "F.Cu") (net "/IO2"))
 (via (at 34.65 33) (size 0.6) (drill 0.3) (layers "F.Cu" "B.Cu") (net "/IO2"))
 (segment (start 34.65 33) (end 42.675 24.975) (width 0.2) (layer "B.Cu") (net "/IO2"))
 (segment (start 42.675 24.975) (end 42.75 24.975) (width 0.2) (layer "B.Cu") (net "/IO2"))
 (segment (start 42.75 24.975) (end 42.78 25) (width 0.2) (layer "B.Cu") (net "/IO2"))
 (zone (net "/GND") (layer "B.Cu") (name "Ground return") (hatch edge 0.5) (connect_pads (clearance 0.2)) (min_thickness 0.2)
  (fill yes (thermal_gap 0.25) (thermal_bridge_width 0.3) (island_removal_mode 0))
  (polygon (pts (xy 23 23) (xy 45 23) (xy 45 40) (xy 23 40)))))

